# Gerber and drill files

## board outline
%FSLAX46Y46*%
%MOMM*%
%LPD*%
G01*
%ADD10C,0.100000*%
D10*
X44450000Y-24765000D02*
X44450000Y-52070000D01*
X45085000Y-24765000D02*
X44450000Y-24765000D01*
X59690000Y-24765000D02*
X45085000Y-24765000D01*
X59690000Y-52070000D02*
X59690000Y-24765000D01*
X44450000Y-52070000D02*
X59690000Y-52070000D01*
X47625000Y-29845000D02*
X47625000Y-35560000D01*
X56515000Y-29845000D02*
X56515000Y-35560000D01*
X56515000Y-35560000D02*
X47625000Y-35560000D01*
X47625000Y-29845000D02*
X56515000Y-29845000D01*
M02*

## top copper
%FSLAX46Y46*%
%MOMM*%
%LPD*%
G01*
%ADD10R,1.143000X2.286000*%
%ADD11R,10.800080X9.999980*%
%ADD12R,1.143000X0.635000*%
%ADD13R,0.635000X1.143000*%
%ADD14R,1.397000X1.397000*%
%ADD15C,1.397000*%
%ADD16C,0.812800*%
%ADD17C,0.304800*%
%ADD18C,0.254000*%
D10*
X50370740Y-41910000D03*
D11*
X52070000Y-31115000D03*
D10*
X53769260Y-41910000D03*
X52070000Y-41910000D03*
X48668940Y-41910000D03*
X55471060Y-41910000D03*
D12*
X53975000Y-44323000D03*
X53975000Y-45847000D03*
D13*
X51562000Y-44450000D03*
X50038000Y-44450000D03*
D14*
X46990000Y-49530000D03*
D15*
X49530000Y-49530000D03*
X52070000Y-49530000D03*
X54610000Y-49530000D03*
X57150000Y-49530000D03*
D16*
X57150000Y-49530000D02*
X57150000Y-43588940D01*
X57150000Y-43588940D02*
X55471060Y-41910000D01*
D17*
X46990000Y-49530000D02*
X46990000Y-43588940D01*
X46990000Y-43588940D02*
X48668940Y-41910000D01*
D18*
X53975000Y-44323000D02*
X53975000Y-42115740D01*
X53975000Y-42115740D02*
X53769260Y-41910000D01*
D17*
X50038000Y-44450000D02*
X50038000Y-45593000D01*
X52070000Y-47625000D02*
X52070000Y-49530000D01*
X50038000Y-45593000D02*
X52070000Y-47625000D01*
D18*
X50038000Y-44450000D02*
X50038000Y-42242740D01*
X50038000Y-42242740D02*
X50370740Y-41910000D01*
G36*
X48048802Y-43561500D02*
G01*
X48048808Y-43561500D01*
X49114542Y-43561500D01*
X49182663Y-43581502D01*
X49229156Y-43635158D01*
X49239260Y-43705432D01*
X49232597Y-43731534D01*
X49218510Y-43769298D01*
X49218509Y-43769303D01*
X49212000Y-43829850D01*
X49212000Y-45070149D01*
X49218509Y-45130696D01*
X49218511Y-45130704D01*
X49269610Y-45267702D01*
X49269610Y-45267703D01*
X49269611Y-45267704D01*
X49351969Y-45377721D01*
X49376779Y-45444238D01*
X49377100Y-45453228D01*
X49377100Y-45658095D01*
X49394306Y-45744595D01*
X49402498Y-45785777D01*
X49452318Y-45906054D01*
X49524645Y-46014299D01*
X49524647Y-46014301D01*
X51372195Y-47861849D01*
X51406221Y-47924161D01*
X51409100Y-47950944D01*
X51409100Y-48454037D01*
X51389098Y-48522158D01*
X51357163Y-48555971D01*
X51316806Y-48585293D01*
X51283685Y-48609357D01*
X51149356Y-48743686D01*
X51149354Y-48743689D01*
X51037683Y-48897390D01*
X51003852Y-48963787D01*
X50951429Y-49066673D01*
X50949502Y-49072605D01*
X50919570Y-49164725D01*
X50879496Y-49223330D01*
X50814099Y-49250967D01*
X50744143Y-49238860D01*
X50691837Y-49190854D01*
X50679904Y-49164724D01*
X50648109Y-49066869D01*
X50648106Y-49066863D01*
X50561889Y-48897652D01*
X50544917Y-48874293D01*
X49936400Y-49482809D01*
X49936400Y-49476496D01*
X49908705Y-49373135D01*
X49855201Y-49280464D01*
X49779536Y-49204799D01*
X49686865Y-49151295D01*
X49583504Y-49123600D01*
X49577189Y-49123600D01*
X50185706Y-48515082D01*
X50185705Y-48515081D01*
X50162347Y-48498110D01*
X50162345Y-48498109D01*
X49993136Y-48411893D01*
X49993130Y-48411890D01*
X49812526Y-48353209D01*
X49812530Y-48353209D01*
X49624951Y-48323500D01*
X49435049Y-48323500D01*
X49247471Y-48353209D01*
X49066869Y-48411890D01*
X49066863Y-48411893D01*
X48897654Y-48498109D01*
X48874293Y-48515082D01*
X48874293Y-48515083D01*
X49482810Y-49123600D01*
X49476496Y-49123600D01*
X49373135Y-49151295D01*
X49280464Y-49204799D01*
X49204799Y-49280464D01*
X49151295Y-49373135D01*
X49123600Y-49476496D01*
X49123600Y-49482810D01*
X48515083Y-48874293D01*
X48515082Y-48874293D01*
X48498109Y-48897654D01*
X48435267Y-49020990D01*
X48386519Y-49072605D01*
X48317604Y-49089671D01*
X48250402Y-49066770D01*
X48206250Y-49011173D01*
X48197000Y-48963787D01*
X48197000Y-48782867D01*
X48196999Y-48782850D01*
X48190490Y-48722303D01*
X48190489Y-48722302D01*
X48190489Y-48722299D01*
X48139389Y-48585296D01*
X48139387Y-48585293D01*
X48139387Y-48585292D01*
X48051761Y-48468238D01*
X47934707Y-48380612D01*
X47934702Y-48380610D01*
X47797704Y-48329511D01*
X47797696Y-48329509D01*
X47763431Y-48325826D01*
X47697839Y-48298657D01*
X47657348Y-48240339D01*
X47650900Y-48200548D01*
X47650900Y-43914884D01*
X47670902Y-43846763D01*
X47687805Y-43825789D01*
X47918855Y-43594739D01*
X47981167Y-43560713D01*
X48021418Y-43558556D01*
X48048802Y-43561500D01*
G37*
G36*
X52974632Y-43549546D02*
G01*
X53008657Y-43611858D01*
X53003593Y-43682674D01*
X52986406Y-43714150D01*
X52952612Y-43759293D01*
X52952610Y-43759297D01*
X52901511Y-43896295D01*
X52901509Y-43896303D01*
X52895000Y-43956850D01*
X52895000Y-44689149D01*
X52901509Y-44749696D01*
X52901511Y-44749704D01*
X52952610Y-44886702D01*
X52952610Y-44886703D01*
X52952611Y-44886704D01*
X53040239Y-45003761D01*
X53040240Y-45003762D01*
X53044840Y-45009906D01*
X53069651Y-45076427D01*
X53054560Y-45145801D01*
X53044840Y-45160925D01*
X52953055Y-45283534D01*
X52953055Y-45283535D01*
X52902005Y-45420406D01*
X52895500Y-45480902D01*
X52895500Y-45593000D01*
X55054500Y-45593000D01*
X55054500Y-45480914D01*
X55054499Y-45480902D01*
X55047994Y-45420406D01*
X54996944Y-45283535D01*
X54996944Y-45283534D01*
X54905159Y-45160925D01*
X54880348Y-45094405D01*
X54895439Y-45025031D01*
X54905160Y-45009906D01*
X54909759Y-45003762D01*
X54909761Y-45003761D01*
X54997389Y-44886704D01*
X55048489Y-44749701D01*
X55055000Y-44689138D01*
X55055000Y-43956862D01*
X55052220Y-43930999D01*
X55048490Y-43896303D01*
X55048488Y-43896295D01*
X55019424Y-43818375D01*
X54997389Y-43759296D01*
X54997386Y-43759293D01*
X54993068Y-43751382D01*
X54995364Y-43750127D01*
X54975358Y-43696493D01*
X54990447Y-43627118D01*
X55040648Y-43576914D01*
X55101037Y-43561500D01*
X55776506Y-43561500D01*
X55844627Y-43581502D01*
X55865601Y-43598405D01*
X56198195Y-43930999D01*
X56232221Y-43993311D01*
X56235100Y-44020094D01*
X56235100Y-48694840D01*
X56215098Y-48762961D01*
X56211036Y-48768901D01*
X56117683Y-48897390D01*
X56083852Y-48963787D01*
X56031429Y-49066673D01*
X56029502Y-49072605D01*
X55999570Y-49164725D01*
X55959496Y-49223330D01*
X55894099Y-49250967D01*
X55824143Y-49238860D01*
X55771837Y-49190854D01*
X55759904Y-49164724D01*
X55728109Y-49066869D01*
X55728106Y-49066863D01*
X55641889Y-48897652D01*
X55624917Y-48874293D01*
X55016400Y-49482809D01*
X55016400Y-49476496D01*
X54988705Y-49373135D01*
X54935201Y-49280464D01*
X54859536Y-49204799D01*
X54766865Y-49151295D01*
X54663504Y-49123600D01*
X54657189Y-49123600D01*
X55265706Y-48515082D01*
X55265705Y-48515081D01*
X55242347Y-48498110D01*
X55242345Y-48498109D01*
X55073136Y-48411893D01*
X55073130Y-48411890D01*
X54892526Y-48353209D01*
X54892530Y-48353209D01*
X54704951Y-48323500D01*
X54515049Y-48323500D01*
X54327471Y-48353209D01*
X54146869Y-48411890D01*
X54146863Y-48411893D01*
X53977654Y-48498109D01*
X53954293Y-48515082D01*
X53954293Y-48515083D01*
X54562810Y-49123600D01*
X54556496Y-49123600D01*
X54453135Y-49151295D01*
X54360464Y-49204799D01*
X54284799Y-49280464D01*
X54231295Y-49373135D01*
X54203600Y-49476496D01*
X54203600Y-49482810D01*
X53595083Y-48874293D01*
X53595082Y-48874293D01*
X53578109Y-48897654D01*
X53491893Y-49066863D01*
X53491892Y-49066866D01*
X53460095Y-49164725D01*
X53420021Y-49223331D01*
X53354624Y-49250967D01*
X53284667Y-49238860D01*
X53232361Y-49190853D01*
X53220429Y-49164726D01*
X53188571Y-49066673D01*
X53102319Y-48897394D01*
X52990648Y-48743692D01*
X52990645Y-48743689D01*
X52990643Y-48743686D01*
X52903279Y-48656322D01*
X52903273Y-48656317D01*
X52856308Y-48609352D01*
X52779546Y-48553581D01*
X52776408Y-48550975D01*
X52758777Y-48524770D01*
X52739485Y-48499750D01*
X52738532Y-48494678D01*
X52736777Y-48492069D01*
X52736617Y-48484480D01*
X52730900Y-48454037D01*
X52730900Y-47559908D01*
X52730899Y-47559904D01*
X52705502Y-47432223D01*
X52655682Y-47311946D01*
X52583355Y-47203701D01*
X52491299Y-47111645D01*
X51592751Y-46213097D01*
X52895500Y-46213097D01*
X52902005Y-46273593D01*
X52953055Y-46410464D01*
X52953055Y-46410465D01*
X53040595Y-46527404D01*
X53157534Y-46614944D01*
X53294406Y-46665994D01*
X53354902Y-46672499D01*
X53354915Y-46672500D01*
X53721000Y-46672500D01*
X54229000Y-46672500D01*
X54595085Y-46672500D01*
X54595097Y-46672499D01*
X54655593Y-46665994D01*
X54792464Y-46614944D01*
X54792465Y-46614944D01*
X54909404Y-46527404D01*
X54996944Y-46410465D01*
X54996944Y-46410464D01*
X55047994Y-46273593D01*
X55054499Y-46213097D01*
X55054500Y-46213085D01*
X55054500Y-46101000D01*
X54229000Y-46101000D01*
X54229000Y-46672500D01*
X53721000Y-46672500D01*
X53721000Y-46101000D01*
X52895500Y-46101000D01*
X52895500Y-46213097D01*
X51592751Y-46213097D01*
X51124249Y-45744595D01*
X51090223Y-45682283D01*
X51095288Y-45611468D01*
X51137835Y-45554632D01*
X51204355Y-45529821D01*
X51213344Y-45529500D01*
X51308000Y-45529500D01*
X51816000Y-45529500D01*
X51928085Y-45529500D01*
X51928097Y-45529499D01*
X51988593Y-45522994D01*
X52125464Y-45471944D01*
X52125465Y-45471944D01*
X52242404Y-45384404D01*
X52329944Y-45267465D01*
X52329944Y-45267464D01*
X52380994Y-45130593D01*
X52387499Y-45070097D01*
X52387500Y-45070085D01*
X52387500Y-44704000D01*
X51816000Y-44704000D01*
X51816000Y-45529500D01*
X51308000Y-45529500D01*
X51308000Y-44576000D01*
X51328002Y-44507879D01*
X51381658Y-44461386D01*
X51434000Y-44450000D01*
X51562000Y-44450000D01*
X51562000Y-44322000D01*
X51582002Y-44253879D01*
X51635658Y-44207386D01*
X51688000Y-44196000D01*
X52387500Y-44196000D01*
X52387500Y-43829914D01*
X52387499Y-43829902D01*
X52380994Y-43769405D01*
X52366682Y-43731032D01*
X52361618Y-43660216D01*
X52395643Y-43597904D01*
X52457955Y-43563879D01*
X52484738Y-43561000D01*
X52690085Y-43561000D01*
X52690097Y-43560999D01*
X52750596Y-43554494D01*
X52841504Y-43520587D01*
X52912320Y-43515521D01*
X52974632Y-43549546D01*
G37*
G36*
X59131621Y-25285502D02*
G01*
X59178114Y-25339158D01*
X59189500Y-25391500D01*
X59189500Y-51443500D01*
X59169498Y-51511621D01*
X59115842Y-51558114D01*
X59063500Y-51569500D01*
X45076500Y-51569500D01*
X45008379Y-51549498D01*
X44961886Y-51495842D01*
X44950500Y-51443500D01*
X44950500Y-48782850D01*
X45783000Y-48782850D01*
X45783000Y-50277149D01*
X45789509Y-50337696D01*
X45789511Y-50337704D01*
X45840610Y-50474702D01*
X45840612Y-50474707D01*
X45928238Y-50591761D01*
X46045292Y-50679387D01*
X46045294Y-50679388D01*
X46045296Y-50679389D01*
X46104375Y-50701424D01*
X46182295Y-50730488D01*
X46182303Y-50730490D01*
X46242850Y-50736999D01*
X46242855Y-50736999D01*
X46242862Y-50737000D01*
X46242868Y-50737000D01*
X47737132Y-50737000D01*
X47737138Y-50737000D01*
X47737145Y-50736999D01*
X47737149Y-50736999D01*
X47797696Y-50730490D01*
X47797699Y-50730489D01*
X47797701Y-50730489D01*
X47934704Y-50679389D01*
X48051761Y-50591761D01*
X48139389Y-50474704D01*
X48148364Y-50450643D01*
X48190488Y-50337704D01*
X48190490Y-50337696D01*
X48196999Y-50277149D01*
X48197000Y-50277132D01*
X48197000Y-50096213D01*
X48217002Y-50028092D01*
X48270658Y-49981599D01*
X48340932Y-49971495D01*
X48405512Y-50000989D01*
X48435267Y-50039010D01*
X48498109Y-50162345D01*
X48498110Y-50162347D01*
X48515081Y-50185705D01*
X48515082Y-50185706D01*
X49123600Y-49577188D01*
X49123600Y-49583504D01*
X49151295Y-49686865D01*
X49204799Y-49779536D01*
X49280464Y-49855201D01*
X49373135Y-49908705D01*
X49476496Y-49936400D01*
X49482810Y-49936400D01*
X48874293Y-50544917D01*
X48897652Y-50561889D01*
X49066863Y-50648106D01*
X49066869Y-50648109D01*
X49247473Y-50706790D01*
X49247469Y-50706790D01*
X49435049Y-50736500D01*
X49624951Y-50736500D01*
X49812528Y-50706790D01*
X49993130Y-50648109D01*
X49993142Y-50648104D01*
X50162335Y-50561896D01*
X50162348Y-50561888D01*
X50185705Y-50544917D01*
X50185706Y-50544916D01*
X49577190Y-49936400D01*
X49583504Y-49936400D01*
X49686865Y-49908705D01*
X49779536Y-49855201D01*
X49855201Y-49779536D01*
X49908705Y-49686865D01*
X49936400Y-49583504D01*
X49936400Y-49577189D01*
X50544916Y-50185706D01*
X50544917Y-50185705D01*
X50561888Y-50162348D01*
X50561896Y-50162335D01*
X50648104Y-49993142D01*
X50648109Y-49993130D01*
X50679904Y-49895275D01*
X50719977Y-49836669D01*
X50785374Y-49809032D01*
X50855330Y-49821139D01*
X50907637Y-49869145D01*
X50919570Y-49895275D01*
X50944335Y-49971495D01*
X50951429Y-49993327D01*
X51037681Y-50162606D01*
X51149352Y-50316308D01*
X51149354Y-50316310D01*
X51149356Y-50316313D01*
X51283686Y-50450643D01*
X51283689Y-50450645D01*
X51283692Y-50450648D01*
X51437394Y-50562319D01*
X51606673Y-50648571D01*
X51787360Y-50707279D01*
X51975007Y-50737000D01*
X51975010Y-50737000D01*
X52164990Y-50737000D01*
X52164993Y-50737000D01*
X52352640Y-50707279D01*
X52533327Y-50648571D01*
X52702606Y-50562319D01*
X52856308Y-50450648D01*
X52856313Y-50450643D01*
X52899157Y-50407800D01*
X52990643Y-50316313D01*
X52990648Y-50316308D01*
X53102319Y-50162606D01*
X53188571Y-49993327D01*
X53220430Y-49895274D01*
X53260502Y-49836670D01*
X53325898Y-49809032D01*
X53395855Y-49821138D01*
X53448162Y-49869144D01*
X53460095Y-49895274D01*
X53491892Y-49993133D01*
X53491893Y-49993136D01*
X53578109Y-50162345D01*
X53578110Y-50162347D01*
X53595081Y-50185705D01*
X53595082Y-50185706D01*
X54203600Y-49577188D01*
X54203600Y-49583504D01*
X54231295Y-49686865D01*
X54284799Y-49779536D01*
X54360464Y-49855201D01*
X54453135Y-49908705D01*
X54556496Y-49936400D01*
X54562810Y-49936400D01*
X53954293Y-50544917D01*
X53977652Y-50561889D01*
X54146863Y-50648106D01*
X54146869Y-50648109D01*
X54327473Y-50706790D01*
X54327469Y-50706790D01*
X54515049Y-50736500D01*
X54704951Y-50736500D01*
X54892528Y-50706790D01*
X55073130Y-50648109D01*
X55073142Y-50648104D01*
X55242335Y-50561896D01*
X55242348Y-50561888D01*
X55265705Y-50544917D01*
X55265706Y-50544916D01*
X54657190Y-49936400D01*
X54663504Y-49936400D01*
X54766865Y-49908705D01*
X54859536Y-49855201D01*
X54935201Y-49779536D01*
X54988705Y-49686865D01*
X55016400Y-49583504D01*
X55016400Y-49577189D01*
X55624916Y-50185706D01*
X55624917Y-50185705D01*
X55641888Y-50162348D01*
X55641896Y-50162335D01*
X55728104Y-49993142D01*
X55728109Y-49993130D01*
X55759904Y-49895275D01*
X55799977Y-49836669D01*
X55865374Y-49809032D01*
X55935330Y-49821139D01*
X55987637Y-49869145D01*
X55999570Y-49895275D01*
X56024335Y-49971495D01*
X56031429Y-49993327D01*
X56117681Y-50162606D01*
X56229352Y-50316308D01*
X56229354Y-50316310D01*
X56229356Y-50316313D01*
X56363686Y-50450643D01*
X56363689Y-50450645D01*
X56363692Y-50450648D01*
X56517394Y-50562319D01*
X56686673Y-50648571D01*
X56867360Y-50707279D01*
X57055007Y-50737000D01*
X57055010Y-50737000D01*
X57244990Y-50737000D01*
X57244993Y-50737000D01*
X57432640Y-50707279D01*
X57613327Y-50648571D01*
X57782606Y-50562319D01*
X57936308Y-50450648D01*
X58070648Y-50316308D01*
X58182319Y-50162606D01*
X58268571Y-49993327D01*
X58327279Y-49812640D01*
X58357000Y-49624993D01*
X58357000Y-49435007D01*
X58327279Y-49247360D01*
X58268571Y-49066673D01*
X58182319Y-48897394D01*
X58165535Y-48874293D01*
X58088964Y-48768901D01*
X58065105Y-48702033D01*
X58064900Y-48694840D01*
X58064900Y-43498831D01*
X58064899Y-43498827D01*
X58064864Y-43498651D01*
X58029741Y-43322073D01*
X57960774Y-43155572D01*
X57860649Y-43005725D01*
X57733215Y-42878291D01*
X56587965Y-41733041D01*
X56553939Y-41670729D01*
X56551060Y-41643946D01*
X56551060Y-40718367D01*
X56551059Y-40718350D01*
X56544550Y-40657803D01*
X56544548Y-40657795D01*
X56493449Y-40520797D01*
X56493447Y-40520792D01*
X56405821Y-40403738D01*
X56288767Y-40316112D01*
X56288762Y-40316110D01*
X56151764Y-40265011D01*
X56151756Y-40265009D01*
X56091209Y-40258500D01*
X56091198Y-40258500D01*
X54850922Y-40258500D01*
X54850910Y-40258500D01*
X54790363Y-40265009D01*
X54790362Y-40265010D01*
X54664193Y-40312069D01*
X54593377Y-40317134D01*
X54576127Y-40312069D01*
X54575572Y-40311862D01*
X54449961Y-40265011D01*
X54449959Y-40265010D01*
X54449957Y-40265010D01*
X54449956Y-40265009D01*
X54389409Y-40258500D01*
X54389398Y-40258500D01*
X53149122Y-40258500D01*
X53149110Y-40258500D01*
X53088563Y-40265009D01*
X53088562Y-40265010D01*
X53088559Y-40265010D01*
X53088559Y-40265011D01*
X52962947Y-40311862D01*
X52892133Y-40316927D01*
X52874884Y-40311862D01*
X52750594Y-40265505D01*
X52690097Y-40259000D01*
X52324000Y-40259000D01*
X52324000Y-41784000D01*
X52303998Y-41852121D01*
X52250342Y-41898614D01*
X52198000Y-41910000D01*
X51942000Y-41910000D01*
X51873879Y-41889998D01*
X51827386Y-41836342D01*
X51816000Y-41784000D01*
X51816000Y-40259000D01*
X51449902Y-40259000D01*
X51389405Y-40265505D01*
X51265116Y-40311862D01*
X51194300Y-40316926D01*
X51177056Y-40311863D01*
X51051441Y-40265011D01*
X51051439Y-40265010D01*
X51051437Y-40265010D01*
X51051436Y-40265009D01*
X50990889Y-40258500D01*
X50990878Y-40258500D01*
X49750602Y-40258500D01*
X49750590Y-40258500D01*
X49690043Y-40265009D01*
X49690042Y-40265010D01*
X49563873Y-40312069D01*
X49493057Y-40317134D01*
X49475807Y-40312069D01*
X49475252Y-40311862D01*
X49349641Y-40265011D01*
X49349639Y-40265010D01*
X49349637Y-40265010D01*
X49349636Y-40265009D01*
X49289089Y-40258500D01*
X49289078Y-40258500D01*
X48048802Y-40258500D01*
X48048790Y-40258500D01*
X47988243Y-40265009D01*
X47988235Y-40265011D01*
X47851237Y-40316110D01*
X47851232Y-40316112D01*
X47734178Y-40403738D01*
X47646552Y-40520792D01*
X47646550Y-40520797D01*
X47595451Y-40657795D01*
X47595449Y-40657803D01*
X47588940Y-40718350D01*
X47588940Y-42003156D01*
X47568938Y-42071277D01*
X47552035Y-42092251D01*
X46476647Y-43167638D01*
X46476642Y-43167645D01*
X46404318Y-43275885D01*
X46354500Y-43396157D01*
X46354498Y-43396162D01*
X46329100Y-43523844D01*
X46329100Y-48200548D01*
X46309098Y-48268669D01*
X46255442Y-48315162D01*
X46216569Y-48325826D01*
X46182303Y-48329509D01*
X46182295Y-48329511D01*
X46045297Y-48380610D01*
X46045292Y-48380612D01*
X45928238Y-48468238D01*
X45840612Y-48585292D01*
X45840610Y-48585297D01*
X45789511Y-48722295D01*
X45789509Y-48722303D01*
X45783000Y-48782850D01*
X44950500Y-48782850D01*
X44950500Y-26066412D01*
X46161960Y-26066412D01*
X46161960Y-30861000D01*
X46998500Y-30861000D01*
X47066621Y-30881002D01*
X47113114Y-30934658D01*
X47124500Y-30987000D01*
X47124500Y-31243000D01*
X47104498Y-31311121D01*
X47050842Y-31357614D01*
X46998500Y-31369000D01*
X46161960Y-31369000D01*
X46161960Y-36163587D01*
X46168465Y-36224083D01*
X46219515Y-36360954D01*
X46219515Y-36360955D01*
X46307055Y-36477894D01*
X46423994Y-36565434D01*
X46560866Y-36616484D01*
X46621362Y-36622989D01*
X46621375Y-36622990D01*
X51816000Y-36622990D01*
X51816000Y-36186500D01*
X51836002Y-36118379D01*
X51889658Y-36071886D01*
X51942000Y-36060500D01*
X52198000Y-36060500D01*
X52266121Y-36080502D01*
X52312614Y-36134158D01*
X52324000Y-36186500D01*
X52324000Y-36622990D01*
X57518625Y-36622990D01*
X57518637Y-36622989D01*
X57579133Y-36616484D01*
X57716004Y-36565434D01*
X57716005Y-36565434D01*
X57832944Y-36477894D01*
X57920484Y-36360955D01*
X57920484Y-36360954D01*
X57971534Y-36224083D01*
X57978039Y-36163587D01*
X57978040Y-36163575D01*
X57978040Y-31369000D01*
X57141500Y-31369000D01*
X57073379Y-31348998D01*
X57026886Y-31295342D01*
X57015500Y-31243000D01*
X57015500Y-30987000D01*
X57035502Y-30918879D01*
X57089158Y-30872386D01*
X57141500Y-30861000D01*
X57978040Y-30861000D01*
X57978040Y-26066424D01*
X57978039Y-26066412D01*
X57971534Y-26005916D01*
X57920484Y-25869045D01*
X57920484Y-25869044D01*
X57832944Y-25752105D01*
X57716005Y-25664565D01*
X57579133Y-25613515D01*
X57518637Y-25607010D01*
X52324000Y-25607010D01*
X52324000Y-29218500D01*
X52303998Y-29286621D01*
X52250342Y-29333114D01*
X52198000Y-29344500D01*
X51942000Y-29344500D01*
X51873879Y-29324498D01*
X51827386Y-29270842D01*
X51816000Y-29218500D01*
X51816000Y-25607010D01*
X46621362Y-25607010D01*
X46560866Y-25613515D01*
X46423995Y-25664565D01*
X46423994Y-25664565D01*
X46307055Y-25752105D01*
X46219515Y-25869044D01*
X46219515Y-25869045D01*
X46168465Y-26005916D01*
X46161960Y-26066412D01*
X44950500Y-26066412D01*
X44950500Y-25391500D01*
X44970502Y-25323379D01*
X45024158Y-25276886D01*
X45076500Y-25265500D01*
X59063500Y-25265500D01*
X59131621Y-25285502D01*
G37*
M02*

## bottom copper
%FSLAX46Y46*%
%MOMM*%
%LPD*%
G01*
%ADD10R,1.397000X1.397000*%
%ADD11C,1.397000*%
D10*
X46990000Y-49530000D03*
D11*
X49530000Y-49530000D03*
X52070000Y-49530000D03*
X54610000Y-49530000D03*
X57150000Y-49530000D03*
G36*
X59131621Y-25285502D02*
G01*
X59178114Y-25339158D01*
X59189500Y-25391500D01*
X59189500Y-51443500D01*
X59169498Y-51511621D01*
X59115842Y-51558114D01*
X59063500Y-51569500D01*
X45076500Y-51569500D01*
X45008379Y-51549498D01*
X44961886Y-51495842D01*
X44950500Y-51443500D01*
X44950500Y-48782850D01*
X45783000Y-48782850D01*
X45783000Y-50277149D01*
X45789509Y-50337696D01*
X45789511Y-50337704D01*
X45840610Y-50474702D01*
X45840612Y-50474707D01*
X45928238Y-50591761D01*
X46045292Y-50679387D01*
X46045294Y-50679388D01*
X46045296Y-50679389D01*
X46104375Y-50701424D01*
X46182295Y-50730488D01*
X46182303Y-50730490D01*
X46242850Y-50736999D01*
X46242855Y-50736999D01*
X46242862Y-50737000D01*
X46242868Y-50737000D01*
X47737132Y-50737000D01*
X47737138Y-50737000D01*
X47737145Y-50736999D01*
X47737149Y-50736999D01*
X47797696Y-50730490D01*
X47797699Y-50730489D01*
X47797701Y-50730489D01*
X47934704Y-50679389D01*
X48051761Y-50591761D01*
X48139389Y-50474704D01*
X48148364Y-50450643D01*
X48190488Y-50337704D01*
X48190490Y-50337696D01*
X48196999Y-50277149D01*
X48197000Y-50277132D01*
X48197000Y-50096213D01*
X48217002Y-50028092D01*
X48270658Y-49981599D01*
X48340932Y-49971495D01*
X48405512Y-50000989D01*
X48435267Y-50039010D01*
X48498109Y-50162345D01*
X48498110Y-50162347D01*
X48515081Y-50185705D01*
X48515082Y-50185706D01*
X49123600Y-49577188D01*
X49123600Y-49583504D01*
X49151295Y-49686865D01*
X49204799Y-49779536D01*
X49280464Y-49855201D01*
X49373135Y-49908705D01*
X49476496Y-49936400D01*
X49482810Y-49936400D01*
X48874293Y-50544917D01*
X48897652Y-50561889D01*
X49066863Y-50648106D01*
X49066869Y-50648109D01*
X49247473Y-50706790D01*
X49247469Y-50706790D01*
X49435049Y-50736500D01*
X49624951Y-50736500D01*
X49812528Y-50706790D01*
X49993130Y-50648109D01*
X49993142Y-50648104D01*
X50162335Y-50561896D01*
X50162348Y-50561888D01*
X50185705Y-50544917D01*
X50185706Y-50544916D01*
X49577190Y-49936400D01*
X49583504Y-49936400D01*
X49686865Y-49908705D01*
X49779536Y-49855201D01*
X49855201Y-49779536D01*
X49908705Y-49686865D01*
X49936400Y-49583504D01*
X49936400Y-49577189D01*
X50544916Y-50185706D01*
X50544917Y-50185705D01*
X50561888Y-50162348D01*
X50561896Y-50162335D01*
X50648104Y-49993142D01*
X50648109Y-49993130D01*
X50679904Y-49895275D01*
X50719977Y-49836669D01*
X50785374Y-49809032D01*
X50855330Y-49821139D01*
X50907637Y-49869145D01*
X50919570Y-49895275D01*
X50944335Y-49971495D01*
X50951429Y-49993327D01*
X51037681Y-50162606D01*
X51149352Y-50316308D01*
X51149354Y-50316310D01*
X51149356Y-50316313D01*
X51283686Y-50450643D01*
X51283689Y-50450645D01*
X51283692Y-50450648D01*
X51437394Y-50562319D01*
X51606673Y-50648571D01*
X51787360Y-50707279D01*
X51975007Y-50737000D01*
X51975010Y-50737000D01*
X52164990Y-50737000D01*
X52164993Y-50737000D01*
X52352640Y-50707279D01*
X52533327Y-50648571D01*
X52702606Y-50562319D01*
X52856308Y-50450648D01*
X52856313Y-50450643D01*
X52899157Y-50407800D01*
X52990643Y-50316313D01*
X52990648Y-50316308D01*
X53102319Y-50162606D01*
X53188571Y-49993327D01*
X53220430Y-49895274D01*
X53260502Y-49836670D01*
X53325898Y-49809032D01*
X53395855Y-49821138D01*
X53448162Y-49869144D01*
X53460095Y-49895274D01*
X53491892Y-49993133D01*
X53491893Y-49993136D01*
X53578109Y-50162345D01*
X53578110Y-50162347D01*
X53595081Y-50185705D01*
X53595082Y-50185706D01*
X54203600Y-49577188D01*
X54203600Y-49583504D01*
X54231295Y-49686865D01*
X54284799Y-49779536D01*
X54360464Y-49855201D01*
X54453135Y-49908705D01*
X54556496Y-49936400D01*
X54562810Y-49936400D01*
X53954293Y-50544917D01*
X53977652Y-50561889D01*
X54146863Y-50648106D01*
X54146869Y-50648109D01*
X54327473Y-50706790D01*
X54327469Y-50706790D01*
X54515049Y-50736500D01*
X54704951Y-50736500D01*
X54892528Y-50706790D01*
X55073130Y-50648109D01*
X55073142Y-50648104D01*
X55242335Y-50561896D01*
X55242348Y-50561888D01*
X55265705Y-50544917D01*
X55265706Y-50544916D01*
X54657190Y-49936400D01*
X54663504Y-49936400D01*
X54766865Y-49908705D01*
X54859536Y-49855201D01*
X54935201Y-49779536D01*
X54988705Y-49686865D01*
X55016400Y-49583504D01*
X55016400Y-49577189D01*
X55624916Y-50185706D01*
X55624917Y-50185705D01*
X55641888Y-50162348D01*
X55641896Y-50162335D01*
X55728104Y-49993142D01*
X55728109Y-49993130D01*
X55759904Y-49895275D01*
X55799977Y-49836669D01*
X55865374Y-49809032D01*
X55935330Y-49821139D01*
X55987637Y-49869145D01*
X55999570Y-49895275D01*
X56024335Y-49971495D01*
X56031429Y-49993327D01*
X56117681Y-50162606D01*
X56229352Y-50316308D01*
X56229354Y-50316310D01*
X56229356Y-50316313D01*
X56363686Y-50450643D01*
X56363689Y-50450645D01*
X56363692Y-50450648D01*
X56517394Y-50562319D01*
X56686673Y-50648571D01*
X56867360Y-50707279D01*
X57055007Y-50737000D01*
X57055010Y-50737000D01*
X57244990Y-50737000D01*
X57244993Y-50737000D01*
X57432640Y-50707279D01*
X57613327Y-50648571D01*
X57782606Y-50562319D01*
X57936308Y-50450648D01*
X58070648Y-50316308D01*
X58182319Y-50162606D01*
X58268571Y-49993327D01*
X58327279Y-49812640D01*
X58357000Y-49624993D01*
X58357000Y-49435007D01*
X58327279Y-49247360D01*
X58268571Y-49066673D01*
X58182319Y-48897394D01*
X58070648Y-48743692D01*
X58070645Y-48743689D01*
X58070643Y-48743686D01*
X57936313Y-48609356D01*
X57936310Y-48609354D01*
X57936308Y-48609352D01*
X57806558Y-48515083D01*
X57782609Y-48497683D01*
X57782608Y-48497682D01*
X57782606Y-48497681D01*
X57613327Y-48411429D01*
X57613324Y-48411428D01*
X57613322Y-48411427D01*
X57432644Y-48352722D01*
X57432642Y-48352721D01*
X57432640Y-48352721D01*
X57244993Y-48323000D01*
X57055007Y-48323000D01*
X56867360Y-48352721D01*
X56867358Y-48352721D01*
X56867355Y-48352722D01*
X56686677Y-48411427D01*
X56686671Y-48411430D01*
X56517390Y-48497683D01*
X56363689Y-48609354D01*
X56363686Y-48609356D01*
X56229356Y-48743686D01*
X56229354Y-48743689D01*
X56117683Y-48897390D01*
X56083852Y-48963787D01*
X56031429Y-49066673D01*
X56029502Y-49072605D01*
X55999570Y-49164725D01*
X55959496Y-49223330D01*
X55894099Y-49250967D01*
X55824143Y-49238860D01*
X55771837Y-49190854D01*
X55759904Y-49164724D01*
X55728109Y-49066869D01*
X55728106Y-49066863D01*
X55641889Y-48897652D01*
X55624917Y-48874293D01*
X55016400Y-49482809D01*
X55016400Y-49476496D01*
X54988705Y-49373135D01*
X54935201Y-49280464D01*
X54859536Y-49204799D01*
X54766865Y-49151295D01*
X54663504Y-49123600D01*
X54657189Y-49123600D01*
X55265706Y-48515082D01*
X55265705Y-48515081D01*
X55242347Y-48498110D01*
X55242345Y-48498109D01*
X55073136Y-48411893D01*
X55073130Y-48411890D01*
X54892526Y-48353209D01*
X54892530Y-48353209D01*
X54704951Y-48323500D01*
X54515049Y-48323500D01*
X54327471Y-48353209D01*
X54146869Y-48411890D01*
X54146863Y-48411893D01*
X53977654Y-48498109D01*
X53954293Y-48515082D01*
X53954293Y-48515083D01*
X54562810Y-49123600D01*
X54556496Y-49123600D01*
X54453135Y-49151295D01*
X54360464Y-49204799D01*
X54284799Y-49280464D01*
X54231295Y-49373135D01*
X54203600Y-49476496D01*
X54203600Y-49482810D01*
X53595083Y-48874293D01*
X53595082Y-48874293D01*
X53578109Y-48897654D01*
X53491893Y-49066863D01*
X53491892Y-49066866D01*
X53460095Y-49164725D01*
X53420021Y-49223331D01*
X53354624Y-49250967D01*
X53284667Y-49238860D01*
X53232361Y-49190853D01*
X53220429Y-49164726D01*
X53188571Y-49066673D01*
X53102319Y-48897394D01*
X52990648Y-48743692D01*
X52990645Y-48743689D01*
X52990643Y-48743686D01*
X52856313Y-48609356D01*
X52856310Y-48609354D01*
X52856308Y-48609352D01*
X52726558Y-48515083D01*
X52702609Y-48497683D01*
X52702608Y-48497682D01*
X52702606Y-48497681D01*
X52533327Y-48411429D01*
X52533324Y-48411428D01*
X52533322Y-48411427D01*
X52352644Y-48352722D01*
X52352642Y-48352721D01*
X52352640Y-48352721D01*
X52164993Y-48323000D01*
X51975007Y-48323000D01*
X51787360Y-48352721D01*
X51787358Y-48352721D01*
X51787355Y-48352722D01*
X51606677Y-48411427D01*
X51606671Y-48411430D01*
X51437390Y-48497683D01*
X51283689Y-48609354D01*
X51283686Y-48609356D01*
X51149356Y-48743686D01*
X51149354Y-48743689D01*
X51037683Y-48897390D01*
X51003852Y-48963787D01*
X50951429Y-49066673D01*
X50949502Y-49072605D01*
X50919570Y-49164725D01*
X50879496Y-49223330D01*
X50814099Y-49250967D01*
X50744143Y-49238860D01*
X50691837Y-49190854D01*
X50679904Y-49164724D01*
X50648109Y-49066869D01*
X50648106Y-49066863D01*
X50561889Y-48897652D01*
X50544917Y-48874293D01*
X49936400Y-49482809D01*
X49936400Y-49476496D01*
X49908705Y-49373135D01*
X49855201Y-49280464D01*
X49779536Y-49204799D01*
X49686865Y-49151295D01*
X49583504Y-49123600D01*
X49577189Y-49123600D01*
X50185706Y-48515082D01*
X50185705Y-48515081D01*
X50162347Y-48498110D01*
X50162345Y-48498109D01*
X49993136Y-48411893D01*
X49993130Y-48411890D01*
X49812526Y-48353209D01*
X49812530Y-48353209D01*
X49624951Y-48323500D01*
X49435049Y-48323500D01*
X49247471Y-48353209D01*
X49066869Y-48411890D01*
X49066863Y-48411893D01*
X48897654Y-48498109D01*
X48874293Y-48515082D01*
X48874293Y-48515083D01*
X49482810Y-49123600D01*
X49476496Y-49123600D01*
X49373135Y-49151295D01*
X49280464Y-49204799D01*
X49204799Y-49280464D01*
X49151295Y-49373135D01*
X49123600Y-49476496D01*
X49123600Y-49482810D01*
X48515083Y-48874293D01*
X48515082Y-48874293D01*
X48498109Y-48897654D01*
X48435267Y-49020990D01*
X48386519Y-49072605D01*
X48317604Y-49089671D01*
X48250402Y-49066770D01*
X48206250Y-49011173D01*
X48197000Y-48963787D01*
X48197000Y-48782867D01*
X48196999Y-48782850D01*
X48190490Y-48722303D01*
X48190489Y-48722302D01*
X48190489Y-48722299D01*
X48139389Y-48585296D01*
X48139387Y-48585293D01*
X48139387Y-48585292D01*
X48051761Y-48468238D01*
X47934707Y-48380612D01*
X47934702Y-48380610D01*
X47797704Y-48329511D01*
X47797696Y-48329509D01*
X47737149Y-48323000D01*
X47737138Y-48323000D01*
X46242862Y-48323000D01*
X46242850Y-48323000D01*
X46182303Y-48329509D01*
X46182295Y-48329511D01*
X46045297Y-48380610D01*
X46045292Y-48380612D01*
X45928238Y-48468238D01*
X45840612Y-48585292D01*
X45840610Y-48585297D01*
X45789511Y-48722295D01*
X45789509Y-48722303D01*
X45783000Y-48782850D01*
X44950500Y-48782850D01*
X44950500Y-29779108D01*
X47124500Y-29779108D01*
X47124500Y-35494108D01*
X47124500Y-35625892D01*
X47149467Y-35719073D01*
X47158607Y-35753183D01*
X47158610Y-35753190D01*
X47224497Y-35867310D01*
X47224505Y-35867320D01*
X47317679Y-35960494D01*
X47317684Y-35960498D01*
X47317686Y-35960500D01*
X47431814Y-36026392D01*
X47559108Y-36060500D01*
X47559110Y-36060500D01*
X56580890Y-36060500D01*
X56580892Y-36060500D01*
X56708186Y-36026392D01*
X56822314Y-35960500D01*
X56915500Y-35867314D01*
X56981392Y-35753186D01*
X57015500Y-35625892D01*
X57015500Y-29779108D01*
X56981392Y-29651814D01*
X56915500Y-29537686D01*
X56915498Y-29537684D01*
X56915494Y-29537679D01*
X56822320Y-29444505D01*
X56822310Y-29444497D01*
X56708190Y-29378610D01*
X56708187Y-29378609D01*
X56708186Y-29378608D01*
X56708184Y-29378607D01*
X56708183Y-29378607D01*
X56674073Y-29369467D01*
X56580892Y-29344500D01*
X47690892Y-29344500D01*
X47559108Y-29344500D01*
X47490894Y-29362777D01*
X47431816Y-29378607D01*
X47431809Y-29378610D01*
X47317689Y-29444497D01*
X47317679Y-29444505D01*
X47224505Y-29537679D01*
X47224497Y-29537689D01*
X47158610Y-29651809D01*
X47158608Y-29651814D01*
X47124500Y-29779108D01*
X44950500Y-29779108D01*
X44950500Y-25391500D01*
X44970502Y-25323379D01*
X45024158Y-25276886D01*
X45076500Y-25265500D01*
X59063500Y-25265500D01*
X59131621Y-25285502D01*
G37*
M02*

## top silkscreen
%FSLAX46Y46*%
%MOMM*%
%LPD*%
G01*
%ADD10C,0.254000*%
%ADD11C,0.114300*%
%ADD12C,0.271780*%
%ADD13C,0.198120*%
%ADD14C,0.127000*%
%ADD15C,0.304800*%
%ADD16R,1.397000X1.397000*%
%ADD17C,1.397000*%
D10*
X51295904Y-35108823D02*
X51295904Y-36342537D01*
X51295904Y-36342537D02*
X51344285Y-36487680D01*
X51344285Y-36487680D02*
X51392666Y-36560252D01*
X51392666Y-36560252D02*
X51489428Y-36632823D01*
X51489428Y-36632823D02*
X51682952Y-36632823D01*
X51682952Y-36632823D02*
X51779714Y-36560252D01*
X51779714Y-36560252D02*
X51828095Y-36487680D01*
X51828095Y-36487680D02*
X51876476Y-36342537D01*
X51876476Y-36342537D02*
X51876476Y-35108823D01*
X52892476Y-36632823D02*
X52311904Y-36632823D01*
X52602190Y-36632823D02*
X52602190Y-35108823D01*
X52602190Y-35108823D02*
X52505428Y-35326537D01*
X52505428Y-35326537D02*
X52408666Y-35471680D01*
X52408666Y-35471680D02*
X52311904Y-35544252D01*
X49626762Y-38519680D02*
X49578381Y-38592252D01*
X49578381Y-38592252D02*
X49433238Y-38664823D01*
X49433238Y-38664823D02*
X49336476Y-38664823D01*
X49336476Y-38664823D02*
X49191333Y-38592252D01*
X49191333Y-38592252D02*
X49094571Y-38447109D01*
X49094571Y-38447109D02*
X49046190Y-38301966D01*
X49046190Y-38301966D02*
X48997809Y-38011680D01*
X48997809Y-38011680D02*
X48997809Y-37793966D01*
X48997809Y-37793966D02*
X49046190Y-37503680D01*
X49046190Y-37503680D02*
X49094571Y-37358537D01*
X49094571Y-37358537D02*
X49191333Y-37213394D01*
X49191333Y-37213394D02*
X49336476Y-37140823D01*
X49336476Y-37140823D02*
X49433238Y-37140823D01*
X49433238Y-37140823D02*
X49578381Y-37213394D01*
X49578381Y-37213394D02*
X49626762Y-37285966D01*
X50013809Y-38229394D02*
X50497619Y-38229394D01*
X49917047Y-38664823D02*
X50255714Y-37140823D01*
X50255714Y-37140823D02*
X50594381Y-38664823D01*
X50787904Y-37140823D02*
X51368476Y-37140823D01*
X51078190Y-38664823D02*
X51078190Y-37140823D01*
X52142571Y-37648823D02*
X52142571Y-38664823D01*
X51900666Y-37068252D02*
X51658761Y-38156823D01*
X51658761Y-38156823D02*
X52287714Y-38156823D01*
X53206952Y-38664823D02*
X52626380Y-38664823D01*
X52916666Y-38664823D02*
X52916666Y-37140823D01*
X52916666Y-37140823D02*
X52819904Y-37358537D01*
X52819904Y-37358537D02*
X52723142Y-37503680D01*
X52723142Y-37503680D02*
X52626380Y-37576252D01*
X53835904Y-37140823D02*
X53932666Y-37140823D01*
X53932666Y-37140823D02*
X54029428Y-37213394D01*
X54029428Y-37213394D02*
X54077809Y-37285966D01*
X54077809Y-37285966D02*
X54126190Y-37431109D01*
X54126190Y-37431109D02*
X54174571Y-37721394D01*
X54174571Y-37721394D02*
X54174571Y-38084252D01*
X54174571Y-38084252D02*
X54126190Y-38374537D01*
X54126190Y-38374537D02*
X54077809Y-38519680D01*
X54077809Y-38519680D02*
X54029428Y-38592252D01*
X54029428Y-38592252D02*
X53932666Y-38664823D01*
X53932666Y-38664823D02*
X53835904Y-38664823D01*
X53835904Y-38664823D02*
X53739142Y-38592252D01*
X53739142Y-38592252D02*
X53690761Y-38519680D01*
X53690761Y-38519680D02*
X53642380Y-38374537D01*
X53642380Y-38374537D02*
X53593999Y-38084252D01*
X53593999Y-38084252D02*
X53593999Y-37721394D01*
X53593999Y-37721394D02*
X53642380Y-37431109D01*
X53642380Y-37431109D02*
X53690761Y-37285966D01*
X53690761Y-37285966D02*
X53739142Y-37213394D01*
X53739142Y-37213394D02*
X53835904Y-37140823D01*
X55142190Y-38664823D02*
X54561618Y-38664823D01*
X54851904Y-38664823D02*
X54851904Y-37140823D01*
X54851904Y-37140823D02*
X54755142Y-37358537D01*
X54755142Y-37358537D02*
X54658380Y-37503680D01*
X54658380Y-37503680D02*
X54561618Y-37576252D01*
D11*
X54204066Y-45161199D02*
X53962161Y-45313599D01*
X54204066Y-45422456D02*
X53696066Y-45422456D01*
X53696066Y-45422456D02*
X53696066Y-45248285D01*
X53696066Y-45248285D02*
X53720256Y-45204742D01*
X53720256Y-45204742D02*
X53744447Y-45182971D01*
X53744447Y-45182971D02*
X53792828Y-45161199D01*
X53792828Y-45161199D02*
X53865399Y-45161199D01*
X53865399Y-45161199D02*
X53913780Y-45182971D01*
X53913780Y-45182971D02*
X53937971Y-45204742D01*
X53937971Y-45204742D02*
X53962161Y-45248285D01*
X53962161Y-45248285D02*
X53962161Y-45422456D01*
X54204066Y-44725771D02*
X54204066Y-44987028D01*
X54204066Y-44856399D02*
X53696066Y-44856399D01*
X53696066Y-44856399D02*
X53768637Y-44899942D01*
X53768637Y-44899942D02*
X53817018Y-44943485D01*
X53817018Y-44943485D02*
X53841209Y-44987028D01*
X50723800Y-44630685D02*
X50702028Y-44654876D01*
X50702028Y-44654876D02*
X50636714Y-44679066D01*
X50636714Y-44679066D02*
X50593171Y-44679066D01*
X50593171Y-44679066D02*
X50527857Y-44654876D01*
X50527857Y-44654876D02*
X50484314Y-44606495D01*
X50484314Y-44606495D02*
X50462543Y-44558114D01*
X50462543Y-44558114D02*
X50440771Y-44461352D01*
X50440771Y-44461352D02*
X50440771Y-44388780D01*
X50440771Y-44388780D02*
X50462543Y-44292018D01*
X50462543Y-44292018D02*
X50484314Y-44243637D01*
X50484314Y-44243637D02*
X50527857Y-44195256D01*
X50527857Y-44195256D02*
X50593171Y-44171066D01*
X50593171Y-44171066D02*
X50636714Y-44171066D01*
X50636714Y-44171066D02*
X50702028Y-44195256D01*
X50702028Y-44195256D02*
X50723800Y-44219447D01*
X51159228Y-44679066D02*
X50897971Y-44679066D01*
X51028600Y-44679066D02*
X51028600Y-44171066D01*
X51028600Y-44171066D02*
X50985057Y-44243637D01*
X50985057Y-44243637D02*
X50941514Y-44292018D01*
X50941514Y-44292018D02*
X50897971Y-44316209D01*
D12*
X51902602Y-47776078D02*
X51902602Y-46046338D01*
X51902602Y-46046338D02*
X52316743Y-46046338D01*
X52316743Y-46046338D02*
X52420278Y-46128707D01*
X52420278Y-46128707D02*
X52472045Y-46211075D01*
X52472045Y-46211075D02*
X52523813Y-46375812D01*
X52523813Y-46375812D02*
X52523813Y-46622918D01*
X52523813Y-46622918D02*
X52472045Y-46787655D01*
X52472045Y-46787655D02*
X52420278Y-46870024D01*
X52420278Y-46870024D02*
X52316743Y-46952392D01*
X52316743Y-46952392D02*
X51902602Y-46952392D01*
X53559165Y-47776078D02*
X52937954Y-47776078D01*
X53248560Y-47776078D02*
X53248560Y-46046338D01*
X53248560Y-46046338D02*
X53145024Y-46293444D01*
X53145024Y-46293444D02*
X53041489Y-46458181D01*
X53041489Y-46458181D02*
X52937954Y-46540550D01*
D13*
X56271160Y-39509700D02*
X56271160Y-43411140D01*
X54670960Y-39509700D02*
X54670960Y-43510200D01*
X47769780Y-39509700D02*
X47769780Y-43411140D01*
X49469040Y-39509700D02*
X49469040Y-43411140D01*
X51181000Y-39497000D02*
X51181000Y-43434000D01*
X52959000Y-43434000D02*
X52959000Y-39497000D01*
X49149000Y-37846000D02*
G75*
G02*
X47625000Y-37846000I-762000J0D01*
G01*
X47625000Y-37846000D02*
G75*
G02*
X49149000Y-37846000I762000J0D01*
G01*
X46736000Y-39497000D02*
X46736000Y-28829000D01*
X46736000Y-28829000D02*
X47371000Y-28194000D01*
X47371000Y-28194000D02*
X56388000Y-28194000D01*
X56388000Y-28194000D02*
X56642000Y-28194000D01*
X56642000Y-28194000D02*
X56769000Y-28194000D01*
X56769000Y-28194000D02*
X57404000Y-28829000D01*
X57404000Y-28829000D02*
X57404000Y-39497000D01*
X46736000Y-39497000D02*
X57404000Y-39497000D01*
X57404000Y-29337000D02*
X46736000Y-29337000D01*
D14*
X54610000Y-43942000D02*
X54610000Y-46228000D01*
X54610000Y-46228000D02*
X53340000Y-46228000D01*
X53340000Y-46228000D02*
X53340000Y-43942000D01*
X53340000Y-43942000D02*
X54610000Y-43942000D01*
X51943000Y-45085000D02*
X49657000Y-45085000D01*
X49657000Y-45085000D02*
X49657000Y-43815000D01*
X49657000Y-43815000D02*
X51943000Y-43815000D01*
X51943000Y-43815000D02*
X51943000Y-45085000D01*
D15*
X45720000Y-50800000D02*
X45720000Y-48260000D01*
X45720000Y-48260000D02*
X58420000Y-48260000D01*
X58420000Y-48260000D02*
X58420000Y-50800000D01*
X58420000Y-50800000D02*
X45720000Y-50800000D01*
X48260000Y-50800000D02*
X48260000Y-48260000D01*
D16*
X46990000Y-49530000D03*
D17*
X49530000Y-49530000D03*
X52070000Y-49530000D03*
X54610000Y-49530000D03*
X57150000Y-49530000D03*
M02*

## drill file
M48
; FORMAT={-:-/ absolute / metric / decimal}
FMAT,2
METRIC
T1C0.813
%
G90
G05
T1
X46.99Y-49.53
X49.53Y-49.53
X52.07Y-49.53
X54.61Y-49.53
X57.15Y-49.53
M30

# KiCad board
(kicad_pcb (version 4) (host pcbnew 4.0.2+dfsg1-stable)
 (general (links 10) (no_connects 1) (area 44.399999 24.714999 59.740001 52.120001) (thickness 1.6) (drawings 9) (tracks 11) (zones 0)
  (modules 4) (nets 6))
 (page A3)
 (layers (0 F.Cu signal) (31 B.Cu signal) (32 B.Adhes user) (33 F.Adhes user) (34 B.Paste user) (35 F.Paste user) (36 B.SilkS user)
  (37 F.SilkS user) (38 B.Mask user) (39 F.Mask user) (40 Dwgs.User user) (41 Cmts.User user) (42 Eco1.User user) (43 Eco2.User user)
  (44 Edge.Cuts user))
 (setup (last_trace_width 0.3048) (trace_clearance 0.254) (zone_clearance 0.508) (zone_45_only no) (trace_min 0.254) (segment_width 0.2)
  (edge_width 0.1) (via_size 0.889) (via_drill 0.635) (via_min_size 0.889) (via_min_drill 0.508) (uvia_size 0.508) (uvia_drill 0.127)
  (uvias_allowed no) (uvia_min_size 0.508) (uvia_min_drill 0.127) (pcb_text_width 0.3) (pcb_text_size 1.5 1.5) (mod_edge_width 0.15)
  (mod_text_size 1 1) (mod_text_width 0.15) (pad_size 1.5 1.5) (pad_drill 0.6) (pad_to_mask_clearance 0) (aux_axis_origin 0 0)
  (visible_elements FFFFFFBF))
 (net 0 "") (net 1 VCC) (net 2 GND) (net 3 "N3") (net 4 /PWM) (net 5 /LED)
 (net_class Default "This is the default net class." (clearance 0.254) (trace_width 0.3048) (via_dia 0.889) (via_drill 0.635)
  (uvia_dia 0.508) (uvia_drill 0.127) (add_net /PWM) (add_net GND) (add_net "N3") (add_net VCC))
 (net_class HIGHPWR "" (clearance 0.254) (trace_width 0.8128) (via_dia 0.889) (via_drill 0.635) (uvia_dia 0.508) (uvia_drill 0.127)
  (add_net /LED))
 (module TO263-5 (layer F.Cu) (at 52.07 41.91)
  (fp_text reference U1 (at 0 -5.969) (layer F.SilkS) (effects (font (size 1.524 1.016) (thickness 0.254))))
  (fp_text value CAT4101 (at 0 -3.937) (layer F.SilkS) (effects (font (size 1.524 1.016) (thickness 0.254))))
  (fp_line (start 4.20116 -2.4003) (end 4.20116 1.50114) (layer F.SilkS) (width 0.19812))
  (fp_line (start 2.60096 -2.4003) (end 2.60096 1.6002) (layer F.SilkS) (width 0.19812))
  (fp_line (start -4.30022 -2.4003) (end -4.30022 1.50114) (layer F.SilkS) (width 0.19812))
  (fp_line (start -2.60096 -2.4003) (end -2.60096 1.50114) (layer F.SilkS) (width 0.19812))
  (fp_line (start -0.889 -2.413) (end -0.889 1.524) (layer F.SilkS) (width 0.19812))
  (fp_line (start 0.889 1.524) (end 0.889 -2.413) (layer F.SilkS) (width 0.19812))
  (fp_circle (center -3.683 -4.064) (end -3.683 -3.302) (layer F.SilkS) (width 0.19812))
  (fp_line (start -5.334 -2.413) (end -5.334 -13.081) (layer F.SilkS) (width 0.19812))
  (fp_line (start -5.334 -13.081) (end -4.699 -13.716) (layer F.SilkS) (width 0.19812))
  (fp_line (start -4.699 -13.716) (end 4.318 -13.716) (layer F.SilkS) (width 0.19812))
  (fp_line (start 4.318 -13.716) (end 4.572 -13.716) (layer F.SilkS) (width 0.19812))
  (fp_line (start 4.572 -13.716) (end 4.699 -13.716) (layer F.SilkS) (width 0.19812))
  (fp_line (start 4.699 -13.716) (end 5.334 -13.081) (layer F.SilkS) (width 0.19812))
  (fp_line (start 5.334 -13.081) (end 5.334 -2.413) (layer F.SilkS) (width 0.19812))
  (fp_line (start -5.334 -2.413) (end 5.334 -2.413) (layer F.SilkS) (width 0.19812))
  (fp_line (start 5.334 -12.573) (end -5.334 -12.573) (layer F.SilkS) (width 0.19812))
  (pad 2 smd rect (at -1.69926 0) (size 1.143 2.286) (layers F.Cu F.Paste F.Mask) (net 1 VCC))
  (pad 3 smd rect (at 0 -10.795) (size 10.80008 9.99998) (layers F.Cu F.Paste F.Mask) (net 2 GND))
  (pad 4 smd rect (at 1.69926 0) (size 1.143 2.286) (layers F.Cu F.Paste F.Mask) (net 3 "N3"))
  (pad 3 smd rect (at 0 0) (size 1.143 2.286) (layers F.Cu F.Paste F.Mask) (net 2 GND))
  (pad 1 smd rect (at -3.40106 0) (size 1.143 2.286) (layers F.Cu F.Paste F.Mask) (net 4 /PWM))
  (pad 5 smd rect (at 3.40106 0) (size 1.143 2.286) (layers F.Cu F.Paste F.Mask) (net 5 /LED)))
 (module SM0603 (layer F.Cu) (at 53.975 45.085 270)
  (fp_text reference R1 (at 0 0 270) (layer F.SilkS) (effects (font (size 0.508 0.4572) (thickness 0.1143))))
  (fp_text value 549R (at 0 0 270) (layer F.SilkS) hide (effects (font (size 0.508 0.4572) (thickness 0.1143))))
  (fp_line (start -1.143 -0.635) (end 1.143 -0.635) (layer F.SilkS) (width 0.127))
  (fp_line (start 1.143 -0.635) (end 1.143 0.635) (layer F.SilkS) (width 0.127))
  (fp_line (start 1.143 0.635) (end -1.143 0.635) (layer F.SilkS) (width 0.127))
  (fp_line (start -1.143 0.635) (end -1.143 -0.635) (layer F.SilkS) (width 0.127))
  (pad 1 smd rect (at -0.762 0 270) (size 0.635 1.143) (layers F.Cu F.Paste F.Mask) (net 3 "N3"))
  (pad 2 smd rect (at 0.762 0 270) (size 0.635 1.143) (layers F.Cu F.Paste F.Mask) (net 2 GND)))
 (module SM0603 (layer F.Cu) (at 50.8 44.45 180)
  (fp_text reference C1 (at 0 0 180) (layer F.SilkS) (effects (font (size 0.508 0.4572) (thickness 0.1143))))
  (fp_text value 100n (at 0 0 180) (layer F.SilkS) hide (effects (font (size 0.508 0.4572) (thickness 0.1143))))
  (fp_line (start -1.143 -0.635) (end 1.143 -0.635) (layer F.SilkS) (width 0.127))
  (fp_line (start 1.143 -0.635) (end 1.143 0.635) (layer F.SilkS) (width 0.127))
  (fp_line (start 1.143 0.635) (end -1.143 0.635) (layer F.SilkS) (width 0.127))
  (fp_line (start -1.143 0.635) (end -1.143 -0.635) (layer F.SilkS) (width 0.127))
  (pad 1 smd rect (at -0.762 0 180) (size 0.635 1.143) (layers F.Cu F.Paste F.Mask) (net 2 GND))
  (pad 2 smd rect (at 0.762 0 180) (size 0.635 1.143) (layers F.Cu F.Paste F.Mask) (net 1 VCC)))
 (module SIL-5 (layer F.Cu) (at 53.34 49.53)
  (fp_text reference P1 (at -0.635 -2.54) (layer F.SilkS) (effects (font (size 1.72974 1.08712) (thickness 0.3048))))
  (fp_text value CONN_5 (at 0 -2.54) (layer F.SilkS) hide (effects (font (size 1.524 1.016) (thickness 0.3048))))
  (fp_line (start -7.62 1.27) (end -7.62 -1.27) (layer F.SilkS) (width 0.3048))
  (fp_line (start -7.62 -1.27) (end 5.08 -1.27) (layer F.SilkS) (width 0.3048))
  (fp_line (start 5.08 -1.27) (end 5.08 1.27) (layer F.SilkS) (width 0.3048))
  (fp_line (start 5.08 1.27) (end -7.62 1.27) (layer F.SilkS) (width 0.3048))
  (fp_line (start -5.08 1.27) (end -5.08 -1.27) (layer F.SilkS) (width 0.3048))
  (pad 1 thru_hole rect (at -6.35 0) (size 1.397 1.397) (drill 0.8128) (layers *.Cu *.Mask F.SilkS) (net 4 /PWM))
  (pad 2 thru_hole circle (at -3.81 0) (size 1.397 1.397) (drill 0.8128) (layers *.Cu *.Mask F.SilkS) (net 2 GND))
  (pad 3 thru_hole circle (at -1.27 0) (size 1.397 1.397) (drill 0.8128) (layers *.Cu *.Mask F.SilkS) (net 1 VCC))
  (pad 4 thru_hole circle (at 1.27 0) (size 1.397 1.397) (drill 0.8128) (layers *.Cu *.Mask F.SilkS) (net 2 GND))
  (pad 5 thru_hole circle (at 3.81 0) (size 1.397 1.397) (drill 0.8128) (layers *.Cu *.Mask F.SilkS) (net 5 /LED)))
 (gr_line (start 44.45 24.765) (end 44.45 52.07) (angle 90) (layer Edge.Cuts) (width 0.1))
 (gr_line (start 45.085 24.765) (end 44.45 24.765) (angle 90) (layer Edge.Cuts) (width 0.1))
 (gr_line (start 59.69 24.765) (end 45.085 24.765) (angle 90) (layer Edge.Cuts) (width 0.1))
 (gr_line (start 59.69 52.07) (end 59.69 24.765) (angle 90) (layer Edge.Cuts) (width 0.1))
 (gr_line (start 44.45 52.07) (end 59.69 52.07) (angle 90) (layer Edge.Cuts) (width 0.1))
 (gr_line (start 47.625 29.845) (end 47.625 35.56) (angle 90) (layer Edge.Cuts) (width 0.1))
 (gr_line (start 56.515 29.845) (end 56.515 35.56) (angle 90) (layer Edge.Cuts) (width 0.1))
 (gr_line (start 56.515 35.56) (end 47.625 35.56) (angle 90) (layer Edge.Cuts) (width 0.1))
 (gr_line (start 47.625 29.845) (end 56.515 29.845) (angle 90) (layer Edge.Cuts) (width 0.1))
 (segment (start 57.15 49.53) (end 57.15 43.58894) (width 0.8128) (layer F.Cu) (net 5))
 (segment (start 57.15 43.58894) (end 55.47106 41.91) (width 0.8128) (layer F.Cu) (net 5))
 (segment (start 46.99 49.53) (end 46.99 43.58894) (width 0.3048) (layer F.Cu) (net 4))
 (segment (start 46.99 43.58894) (end 48.66894 41.91) (width 0.3048) (layer F.Cu) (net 4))
 (segment (start 53.975 44.323) (end 53.975 42.11574) (width 0.254) (layer F.Cu) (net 3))
 (segment (start 53.975 42.11574) (end 53.76926 41.91) (width 0.254) (layer F.Cu) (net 3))
 (segment (start 50.038 44.45) (end 50.038 45.593) (width 0.3048) (layer F.Cu) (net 1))
 (segment (start 52.07 47.625) (end 52.07 49.53) (width 0.3048) (layer F.Cu) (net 1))
 (segment (start 50.038 45.593) (end 52.07 47.625) (width 0.3048) (layer F.Cu) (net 1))
 (segment (start 50.038 44.45) (end 50.038 42.24274) (width 0.254) (layer F.Cu) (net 1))
 (segment (start 50.038 42.24274) (end 50.37074 41.91) (width 0.254) (layer F.Cu) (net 1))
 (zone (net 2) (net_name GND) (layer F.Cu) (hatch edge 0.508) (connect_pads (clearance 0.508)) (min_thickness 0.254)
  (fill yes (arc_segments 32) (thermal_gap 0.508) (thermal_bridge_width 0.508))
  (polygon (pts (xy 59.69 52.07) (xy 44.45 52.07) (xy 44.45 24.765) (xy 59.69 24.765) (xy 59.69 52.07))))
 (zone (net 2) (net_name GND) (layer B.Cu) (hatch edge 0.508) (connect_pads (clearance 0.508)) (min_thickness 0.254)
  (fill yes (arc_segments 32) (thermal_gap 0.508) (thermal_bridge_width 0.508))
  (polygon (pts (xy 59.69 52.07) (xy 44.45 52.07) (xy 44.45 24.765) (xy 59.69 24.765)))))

